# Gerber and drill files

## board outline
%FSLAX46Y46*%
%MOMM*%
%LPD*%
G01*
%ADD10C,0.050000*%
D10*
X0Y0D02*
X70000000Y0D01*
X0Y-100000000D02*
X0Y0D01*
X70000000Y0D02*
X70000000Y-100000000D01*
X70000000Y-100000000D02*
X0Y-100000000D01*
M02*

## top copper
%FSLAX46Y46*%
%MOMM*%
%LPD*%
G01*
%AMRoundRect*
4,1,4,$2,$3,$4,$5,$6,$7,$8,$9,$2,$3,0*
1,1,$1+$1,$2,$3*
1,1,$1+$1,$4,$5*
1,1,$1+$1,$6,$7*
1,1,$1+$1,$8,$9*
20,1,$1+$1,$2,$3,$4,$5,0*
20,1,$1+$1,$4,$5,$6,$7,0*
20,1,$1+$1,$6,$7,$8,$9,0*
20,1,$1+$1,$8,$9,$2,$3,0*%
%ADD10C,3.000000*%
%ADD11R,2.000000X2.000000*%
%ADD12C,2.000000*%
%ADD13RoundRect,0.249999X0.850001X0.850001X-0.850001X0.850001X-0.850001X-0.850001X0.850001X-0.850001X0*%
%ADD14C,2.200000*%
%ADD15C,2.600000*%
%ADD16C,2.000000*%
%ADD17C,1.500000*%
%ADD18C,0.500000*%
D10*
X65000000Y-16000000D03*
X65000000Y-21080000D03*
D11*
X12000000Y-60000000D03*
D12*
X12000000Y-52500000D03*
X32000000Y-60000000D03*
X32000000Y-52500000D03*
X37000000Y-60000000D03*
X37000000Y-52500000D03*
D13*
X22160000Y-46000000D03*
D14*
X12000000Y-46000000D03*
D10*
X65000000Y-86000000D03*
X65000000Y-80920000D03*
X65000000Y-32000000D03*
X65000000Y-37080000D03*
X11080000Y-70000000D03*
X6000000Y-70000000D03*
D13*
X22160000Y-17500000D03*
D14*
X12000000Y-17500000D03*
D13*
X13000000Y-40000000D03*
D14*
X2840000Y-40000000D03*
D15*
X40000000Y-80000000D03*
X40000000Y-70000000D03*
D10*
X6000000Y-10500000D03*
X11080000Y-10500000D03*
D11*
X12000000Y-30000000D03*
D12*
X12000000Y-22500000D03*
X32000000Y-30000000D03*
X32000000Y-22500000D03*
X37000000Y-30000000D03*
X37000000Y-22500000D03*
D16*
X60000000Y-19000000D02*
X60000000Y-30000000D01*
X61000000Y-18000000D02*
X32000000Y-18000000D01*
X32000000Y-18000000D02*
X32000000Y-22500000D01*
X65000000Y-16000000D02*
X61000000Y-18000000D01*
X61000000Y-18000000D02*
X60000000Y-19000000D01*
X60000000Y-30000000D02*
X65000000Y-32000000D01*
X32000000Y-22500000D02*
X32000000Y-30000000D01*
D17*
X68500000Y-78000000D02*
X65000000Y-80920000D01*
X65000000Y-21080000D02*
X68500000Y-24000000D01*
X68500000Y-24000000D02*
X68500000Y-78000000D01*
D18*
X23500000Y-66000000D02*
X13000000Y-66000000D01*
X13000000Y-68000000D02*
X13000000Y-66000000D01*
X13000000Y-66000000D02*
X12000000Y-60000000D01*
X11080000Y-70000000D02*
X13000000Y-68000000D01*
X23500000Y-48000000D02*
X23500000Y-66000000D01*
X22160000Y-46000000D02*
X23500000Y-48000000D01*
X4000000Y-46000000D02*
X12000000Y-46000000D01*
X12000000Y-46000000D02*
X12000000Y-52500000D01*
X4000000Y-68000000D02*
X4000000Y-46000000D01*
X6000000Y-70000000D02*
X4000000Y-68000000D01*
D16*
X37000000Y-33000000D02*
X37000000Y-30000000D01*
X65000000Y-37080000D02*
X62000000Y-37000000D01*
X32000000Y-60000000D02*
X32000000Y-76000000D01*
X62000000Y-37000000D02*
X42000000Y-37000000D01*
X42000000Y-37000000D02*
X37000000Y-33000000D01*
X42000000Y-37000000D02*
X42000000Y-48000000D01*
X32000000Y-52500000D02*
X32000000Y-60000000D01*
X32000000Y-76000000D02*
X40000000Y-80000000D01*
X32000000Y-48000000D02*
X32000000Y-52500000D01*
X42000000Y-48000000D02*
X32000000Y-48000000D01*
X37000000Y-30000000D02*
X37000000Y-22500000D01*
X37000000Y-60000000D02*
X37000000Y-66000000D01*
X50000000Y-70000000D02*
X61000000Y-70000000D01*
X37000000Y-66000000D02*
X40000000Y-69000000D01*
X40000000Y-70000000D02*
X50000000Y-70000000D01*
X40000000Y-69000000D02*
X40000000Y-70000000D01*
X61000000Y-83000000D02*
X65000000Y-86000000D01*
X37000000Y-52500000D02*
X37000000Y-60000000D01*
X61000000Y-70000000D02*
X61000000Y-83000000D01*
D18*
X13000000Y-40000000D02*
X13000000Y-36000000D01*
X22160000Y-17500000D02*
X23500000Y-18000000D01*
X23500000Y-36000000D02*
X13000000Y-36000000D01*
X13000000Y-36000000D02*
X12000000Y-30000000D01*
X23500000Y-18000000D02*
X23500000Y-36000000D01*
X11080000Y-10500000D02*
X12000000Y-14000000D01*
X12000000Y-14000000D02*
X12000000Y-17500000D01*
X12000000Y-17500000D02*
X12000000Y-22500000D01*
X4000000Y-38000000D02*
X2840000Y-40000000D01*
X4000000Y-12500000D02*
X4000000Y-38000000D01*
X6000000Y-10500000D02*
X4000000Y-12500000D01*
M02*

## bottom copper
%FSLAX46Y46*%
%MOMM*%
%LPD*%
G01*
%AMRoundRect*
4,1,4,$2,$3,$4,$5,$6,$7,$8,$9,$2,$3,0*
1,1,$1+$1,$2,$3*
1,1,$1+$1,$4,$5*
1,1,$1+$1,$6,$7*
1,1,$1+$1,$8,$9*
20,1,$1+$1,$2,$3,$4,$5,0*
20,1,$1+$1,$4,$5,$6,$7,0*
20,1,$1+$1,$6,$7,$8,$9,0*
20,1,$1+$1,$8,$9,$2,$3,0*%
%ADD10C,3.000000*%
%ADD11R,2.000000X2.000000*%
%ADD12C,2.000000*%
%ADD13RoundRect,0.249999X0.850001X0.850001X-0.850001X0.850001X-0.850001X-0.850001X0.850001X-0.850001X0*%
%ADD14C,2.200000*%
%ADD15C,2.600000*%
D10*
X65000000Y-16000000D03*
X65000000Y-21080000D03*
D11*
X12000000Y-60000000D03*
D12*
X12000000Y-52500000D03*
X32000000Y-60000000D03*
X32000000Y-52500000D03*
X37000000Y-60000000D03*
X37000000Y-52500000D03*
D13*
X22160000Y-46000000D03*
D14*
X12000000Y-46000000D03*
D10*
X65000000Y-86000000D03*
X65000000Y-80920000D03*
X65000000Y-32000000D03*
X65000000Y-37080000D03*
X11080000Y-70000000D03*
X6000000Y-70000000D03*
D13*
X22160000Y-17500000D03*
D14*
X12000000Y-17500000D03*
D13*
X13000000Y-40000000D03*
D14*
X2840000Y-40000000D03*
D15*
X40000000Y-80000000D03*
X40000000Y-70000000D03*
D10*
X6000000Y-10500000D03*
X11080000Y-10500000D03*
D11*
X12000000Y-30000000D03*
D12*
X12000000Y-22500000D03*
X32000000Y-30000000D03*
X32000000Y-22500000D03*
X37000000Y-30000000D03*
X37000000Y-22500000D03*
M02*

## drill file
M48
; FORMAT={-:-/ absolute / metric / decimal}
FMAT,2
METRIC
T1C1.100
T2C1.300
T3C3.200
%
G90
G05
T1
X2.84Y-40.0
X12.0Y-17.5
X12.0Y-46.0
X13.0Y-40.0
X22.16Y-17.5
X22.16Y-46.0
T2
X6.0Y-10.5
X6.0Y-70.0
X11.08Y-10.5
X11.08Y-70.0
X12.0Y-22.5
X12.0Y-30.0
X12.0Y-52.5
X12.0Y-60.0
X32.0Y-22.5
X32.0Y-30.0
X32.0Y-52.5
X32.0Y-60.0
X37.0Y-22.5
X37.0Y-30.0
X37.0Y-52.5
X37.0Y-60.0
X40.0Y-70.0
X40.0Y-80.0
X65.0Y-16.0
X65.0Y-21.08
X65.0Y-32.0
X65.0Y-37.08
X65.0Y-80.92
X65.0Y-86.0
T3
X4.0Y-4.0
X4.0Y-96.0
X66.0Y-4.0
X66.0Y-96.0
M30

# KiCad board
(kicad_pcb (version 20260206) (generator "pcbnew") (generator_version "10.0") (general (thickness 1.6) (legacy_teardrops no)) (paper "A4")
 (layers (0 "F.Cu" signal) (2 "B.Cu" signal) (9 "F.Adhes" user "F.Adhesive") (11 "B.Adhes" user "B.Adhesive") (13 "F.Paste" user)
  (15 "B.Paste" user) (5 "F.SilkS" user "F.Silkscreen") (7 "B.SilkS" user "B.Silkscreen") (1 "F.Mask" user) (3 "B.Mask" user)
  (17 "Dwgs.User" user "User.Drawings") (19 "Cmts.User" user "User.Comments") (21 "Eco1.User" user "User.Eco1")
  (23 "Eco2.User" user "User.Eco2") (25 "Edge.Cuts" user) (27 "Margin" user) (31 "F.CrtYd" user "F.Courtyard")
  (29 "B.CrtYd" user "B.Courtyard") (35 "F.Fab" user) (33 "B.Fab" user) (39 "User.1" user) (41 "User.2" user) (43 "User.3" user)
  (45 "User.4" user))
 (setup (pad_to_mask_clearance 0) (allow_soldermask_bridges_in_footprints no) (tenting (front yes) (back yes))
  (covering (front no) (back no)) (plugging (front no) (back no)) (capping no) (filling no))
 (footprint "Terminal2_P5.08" (layer "F.Cu") (at 65 16 -90)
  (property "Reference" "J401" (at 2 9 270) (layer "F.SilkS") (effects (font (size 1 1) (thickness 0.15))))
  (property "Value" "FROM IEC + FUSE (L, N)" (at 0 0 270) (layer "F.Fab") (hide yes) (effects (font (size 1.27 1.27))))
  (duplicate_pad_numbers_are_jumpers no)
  (pad "1" thru_hole circle (at 0 0 270) (size 3 3) (drill 1.3) (layers "*.Cu" "*.Mask") (remove_unused_layers no) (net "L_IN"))
  (pad "2" thru_hole circle (at 5.08 0 270) (size 3 3) (drill 1.3) (layers "*.Cu" "*.Mask") (remove_unused_layers no) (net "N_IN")))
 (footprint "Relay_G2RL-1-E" (layer "F.Cu") (at 12 60 90)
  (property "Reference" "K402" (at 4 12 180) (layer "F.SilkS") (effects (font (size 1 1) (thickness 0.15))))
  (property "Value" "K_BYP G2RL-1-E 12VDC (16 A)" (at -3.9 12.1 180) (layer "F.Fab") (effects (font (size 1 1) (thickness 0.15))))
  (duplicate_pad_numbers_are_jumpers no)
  (pad "A1" thru_hole rect (at 0 0 90) (size 2 2) (drill 1.3) (layers "*.Cu" "*.Mask") (remove_unused_layers no) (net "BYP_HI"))
  (pad "A2" thru_hole circle (at 7.5 0 90) (size 2 2) (drill 1.3) (layers "*.Cu" "*.Mask") (remove_unused_layers no) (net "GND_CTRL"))
  (pad "COM" thru_hole circle (at 0 20 90) (size 2 2) (drill 1.3) (layers "*.Cu" "*.Mask") (remove_unused_layers no) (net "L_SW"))
  (pad "COM" thru_hole circle (at 7.5 20 90) (size 2 2) (drill 1.3) (layers "*.Cu" "*.Mask") (remove_unused_layers no) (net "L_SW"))
  (pad "NO" thru_hole circle (at 0 25 90) (size 2 2) (drill 1.3) (layers "*.Cu" "*.Mask") (remove_unused_layers no) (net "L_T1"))
  (pad "NO" thru_hole circle (at 7.5 25 90) (size 2 2) (drill 1.3) (layers "*.Cu" "*.Mask") (remove_unused_layers no) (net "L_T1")))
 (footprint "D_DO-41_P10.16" (layer "F.Cu") (at 22.16 46 180)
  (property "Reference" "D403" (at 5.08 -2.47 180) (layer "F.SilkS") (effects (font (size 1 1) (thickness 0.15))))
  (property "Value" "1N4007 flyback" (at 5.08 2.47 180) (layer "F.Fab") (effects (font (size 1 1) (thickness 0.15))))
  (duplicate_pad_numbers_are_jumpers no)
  (pad "1" thru_hole roundrect (at 0 0 180) (size 2.2 2.2) (drill 1.1) (layers "*.Cu" "*.Mask") (remove_unused_layers no)
   (roundrect_rratio 0.113636) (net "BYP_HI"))
  (pad "2" thru_hole circle (at 10.16 0 180) (size 2.2 2.2) (drill 1.1) (layers "*.Cu" "*.Mask") (remove_unused_layers no) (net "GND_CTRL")))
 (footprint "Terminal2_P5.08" (layer "F.Cu") (at 65 86 90)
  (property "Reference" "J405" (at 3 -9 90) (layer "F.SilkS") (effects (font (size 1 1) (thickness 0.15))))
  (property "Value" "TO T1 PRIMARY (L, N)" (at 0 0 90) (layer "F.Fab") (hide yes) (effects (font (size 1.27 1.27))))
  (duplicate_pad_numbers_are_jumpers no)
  (pad "1" thru_hole circle (at 0 0 90) (size 3 3) (drill 1.3) (layers "*.Cu" "*.Mask") (remove_unused_layers no) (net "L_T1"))
  (pad "2" thru_hole circle (at 5.08 0 90) (size 3 3) (drill 1.3) (layers "*.Cu" "*.Mask") (remove_unused_layers no) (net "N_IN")))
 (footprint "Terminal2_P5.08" (layer "F.Cu") (at 65 32 -90)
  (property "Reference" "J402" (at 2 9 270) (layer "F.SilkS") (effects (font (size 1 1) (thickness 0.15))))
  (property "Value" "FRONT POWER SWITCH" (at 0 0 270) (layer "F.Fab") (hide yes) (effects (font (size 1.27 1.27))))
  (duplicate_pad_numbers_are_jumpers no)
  (pad "1" thru_hole circle (at 0 0 270) (size 3 3) (drill 1.3) (layers "*.Cu" "*.Mask") (remove_unused_layers no) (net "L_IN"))
  (pad "2" thru_hole circle (at 5.08 0 270) (size 3 3) (drill 1.3) (layers "*.Cu" "*.Mask") (remove_unused_layers no) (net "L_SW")))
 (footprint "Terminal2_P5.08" (layer "F.Cu") (at 11.08 70 180)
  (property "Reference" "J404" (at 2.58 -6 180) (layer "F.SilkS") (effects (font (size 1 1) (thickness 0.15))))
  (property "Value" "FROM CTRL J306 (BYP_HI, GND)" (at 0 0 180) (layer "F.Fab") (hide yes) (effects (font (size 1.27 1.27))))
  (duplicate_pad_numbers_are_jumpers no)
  (pad "1" thru_hole circle (at 0 0 180) (size 3 3) (drill 1.3) (layers "*.Cu" "*.Mask") (remove_unused_layers no) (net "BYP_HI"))
  (pad "2" thru_hole circle (at 5.08 0 180) (size 3 3) (drill 1.3) (layers "*.Cu" "*.Mask") (remove_unused_layers no) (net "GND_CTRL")))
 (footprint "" (layer "F.Cu") (at 66 4)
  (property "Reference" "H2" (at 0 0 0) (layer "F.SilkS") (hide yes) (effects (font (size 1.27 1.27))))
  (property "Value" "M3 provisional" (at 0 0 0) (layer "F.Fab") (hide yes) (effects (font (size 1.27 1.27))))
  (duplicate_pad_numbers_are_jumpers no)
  (pad "" np_thru_hole circle (at 0 0) (size 3.2 3.2) (drill 3.2) (layers "*.Cu" "*.Mask")))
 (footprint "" (layer "F.Cu") (at 66 96)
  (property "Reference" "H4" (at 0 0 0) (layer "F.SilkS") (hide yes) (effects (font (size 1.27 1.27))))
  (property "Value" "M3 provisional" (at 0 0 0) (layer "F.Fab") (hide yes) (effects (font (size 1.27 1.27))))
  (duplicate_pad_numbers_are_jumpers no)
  (pad "" np_thru_hole circle (at 0 0) (size 3.2 3.2) (drill 3.2) (layers "*.Cu" "*.Mask")))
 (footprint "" (layer "F.Cu") (at 4 96)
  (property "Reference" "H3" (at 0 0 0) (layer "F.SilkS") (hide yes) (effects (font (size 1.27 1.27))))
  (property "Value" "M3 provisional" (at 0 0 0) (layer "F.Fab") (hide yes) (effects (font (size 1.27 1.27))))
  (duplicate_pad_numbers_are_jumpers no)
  (pad "" np_thru_hole circle (at 0 0) (size 3.2 3.2) (drill 3.2) (layers "*.Cu" "*.Mask")))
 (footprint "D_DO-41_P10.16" (layer "F.Cu") (at 22.16 17.5 180)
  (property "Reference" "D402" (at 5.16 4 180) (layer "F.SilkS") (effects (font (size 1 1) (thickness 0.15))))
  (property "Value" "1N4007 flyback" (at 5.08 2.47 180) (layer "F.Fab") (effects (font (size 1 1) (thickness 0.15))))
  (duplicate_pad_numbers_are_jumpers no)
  (pad "1" thru_hole roundrect (at 0 0 180) (size 2.2 2.2) (drill 1.1) (layers "*.Cu" "*.Mask") (remove_unused_layers no)
   (roundrect_rratio 0.113636) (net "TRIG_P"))
  (pad "2" thru_hole circle (at 10.16 0 180) (size 2.2 2.2) (drill 1.1) (layers "*.Cu" "*.Mask") (remove_unused_layers no) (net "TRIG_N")))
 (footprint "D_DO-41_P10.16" (layer "F.Cu") (at 13 40 180)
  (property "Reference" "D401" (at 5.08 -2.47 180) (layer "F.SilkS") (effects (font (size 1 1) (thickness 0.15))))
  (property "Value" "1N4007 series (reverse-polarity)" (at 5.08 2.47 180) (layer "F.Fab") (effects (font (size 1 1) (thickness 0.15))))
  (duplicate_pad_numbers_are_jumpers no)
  (pad "1" thru_hole roundrect (at 0 0 180) (size 2.2 2.2) (drill 1.1) (layers "*.Cu" "*.Mask") (remove_unused_layers no)
   (roundrect_rratio 0.113636) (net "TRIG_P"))
  (pad "2" thru_hole circle (at 10.16 0 180) (size 2.2 2.2) (drill 1.1) (layers "*.Cu" "*.Mask") (remove_unused_layers no) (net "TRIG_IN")))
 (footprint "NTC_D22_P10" (layer "F.Cu") (at 40 80 90)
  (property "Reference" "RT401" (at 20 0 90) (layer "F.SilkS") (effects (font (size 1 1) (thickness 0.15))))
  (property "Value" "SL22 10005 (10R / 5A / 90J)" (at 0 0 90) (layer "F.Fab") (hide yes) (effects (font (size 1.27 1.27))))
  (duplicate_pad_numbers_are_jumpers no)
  (pad "1" thru_hole circle (at 0 0 90) (size 2.6 2.6) (drill 1.3) (layers "*.Cu" "*.Mask") (remove_unused_layers no) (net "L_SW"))
  (pad "2" thru_hole circle (at 10 0 90) (size 2.6 2.6) (drill 1.3) (layers "*.Cu" "*.Mask") (remove_unused_layers no) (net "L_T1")))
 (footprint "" (layer "F.Cu") (at 4 4)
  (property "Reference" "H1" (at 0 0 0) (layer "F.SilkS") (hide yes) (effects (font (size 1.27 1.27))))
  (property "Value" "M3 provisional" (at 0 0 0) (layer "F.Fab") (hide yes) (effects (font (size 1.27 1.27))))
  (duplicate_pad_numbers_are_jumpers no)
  (pad "" np_thru_hole circle (at 0 0) (size 3.2 3.2) (drill 3.2) (layers "*.Cu" "*.Mask")))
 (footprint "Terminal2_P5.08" (layer "F.Cu") (at 6 10.5)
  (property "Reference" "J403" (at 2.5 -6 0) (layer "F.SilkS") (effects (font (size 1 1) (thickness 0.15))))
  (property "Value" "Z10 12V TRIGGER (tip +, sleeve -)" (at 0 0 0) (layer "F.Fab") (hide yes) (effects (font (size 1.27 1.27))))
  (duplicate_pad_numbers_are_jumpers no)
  (pad "1" thru_hole circle (at 0 0) (size 3 3) (drill 1.3) (layers "*.Cu" "*.Mask") (remove_unused_layers no) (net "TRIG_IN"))
  (pad "2" thru_hole circle (at 5.08 0) (size 3 3) (drill 1.3) (layers "*.Cu" "*.Mask") (remove_unused_layers no) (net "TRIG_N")))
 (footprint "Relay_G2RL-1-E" (layer "F.Cu") (at 12 30 90)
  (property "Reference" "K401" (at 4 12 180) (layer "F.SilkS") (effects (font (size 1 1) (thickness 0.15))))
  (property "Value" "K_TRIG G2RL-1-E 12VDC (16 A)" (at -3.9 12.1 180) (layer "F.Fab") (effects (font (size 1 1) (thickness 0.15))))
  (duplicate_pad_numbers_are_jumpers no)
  (pad "A1" thru_hole rect (at 0 0 90) (size 2 2) (drill 1.3) (layers "*.Cu" "*.Mask") (remove_unused_layers no) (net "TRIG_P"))
  (pad "A2" thru_hole circle (at 7.5 0 90) (size 2 2) (drill 1.3) (layers "*.Cu" "*.Mask") (remove_unused_layers no) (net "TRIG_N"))
  (pad "COM" thru_hole circle (at 0 20 90) (size 2 2) (drill 1.3) (layers "*.Cu" "*.Mask") (remove_unused_layers no) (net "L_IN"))
  (pad "COM" thru_hole circle (at 7.5 20 90) (size 2 2) (drill 1.3) (layers "*.Cu" "*.Mask") (remove_unused_layers no) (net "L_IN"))
  (pad "NO" thru_hole circle (at 0 25 90) (size 2 2) (drill 1.3) (layers "*.Cu" "*.Mask") (remove_unused_layers no) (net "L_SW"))
  (pad "NO" thru_hole circle (at 7.5 25 90) (size 2 2) (drill 1.3) (layers "*.Cu" "*.Mask") (remove_unused_layers no) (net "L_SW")))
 (gr_line (start 0 0) (end 70 0) (stroke (width 0.05) (type default)) (layer "Edge.Cuts"))
 (gr_line (start 0 100) (end 0 0) (stroke (width 0.05) (type default)) (layer "Edge.Cuts"))
 (gr_line (start 70 0) (end 70 100) (stroke (width 0.05) (type default)) (layer "Edge.Cuts"))
 (gr_line (start 70 100) (end 0 100) (stroke (width 0.05) (type default)) (layer "Edge.Cuts"))
 (segment (start 60 19) (end 60 30) (width 2) (layer "F.Cu") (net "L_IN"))
 (segment (start 61 18) (end 32 18) (width 2) (layer "F.Cu") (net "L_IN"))
 (segment (start 32 18) (end 32 22.5) (width 2) (layer "F.Cu") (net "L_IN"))
 (segment (start 65 16) (end 61 18) (width 2) (layer "F.Cu") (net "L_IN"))
 (segment (start 61 18) (end 60 19) (width 2) (layer "F.Cu") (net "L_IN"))
 (segment (start 60 30) (end 65 32) (width 2) (layer "F.Cu") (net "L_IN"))
 (segment (start 32 22.5) (end 32 30) (width 2) (layer "F.Cu") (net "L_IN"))
 (segment (start 68.5 78) (end 65 80.92) (width 1.5) (layer "F.Cu") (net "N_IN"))
 (segment (start 65 21.08) (end 68.5 24) (width 1.5) (layer "F.Cu") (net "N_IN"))
 (segment (start 68.5 24) (end 68.5 78) (width 1.5) (layer "F.Cu") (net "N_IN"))
 (segment (start 23.5 66) (end 13 66) (width 0.5) (layer "F.Cu") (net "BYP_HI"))
 (segment (start 13 68) (end 13 66) (width 0.5) (layer "F.Cu") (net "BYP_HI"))
 (segment (start 13 66) (end 12 60) (width 0.5) (layer "F.Cu") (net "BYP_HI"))
 (segment (start 11.08 70) (end 13 68) (width 0.5) (layer "F.Cu") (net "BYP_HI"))
 (segment (start 23.5 48) (end 23.5 66) (width 0.5) (layer "F.Cu") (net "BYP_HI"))
 (segment (start 22.16 46) (end 23.5 48) (width 0.5) (layer "F.Cu") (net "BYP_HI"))
 (segment (start 4 46) (end 12 46) (width 0.5) (layer "F.Cu") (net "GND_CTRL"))
 (segment (start 12 46) (end 12 52.5) (width 0.5) (layer "F.Cu") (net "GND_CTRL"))
 (segment (start 4 68) (end 4 46) (width 0.5) (layer "F.Cu") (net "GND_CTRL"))
 (segment (start 6 70) (end 4 68) (width 0.5) (layer "F.Cu") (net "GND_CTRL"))
 (segment (start 37 33) (end 37 30) (width 2) (layer "F.Cu") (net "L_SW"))
 (segment (start 65 37.08) (end 62 37) (width 2) (layer "F.Cu") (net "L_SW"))
 (segment (start 32 60) (end 32 76) (width 2) (layer "F.Cu") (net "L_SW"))
 (segment (start 62 37) (end 42 37) (width 2) (layer "F.Cu") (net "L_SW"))
 (segment (start 42 37) (end 37 33) (width 2) (layer "F.Cu") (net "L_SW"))
 (segment (start 42 37) (end 42 48) (width 2) (layer "F.Cu") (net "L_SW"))
 (segment (start 32 52.5) (end 32 60) (width 2) (layer "F.Cu") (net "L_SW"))
 (segment (start 32 76) (end 40 80) (width 2) (layer "F.Cu") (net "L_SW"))
 (segment (start 32 48) (end 32 52.5) (width 2) (layer "F.Cu") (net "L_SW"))
 (segment (start 42 48) (end 32 48) (width 2) (layer "F.Cu") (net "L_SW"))
 (segment (start 37 30) (end 37 22.5) (width 2) (layer "F.Cu") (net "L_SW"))
 (segment (start 37 60) (end 37 66) (width 2) (layer "F.Cu") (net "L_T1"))
 (segment (start 50 70) (end 61 70) (width 2) (layer "F.Cu") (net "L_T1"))
 (segment (start 37 66) (end 40 69) (width 2) (layer "F.Cu") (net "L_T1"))
 (segment (start 40 70) (end 50 70) (width 2) (layer "F.Cu") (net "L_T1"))
 (segment (start 40 69) (end 40 70) (width 2) (layer "F.Cu") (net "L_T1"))
 (segment (start 61 83) (end 65 86) (width 2) (layer "F.Cu") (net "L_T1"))
 (segment (start 37 52.5) (end 37 60) (width 2) (layer "F.Cu") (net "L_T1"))
 (segment (start 61 70) (end 61 83) (width 2) (layer "F.Cu") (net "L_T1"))
 (segment (start 13 40) (end 13 36) (width 0.5) (layer "F.Cu") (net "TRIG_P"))
 (segment (start 22.16 17.5) (end 23.5 18) (width 0.5) (layer "F.Cu") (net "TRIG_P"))
 (segment (start 23.5 36) (end 13 36) (width 0.5) (layer "F.Cu") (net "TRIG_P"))
 (segment (start 13 36) (end 12 30) (width 0.5) (layer "F.Cu") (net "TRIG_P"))
 (segment (start 23.5 18) (end 23.5 36) (width 0.5) (layer "F.Cu") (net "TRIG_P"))
 (segment (start 11.08 10.5) (end 12 14) (width 0.5) (layer "F.Cu") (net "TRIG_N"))
 (segment (start 12 14) (end 12 17.5) (width 0.5) (layer "F.Cu") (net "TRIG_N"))
 (segment (start 12 17.5) (end 12 22.5) (width 0.5) (layer "F.Cu") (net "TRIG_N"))
 (segment (start 4 38) (end 2.84 40) (width 0.5) (layer "F.Cu") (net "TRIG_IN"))
 (segment (start 4 12.5) (end 4 38) (width 0.5) (layer "F.Cu") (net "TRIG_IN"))
 (segment (start 6 10.5) (end 4 12.5) (width 0.5) (layer "F.Cu") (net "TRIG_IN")))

